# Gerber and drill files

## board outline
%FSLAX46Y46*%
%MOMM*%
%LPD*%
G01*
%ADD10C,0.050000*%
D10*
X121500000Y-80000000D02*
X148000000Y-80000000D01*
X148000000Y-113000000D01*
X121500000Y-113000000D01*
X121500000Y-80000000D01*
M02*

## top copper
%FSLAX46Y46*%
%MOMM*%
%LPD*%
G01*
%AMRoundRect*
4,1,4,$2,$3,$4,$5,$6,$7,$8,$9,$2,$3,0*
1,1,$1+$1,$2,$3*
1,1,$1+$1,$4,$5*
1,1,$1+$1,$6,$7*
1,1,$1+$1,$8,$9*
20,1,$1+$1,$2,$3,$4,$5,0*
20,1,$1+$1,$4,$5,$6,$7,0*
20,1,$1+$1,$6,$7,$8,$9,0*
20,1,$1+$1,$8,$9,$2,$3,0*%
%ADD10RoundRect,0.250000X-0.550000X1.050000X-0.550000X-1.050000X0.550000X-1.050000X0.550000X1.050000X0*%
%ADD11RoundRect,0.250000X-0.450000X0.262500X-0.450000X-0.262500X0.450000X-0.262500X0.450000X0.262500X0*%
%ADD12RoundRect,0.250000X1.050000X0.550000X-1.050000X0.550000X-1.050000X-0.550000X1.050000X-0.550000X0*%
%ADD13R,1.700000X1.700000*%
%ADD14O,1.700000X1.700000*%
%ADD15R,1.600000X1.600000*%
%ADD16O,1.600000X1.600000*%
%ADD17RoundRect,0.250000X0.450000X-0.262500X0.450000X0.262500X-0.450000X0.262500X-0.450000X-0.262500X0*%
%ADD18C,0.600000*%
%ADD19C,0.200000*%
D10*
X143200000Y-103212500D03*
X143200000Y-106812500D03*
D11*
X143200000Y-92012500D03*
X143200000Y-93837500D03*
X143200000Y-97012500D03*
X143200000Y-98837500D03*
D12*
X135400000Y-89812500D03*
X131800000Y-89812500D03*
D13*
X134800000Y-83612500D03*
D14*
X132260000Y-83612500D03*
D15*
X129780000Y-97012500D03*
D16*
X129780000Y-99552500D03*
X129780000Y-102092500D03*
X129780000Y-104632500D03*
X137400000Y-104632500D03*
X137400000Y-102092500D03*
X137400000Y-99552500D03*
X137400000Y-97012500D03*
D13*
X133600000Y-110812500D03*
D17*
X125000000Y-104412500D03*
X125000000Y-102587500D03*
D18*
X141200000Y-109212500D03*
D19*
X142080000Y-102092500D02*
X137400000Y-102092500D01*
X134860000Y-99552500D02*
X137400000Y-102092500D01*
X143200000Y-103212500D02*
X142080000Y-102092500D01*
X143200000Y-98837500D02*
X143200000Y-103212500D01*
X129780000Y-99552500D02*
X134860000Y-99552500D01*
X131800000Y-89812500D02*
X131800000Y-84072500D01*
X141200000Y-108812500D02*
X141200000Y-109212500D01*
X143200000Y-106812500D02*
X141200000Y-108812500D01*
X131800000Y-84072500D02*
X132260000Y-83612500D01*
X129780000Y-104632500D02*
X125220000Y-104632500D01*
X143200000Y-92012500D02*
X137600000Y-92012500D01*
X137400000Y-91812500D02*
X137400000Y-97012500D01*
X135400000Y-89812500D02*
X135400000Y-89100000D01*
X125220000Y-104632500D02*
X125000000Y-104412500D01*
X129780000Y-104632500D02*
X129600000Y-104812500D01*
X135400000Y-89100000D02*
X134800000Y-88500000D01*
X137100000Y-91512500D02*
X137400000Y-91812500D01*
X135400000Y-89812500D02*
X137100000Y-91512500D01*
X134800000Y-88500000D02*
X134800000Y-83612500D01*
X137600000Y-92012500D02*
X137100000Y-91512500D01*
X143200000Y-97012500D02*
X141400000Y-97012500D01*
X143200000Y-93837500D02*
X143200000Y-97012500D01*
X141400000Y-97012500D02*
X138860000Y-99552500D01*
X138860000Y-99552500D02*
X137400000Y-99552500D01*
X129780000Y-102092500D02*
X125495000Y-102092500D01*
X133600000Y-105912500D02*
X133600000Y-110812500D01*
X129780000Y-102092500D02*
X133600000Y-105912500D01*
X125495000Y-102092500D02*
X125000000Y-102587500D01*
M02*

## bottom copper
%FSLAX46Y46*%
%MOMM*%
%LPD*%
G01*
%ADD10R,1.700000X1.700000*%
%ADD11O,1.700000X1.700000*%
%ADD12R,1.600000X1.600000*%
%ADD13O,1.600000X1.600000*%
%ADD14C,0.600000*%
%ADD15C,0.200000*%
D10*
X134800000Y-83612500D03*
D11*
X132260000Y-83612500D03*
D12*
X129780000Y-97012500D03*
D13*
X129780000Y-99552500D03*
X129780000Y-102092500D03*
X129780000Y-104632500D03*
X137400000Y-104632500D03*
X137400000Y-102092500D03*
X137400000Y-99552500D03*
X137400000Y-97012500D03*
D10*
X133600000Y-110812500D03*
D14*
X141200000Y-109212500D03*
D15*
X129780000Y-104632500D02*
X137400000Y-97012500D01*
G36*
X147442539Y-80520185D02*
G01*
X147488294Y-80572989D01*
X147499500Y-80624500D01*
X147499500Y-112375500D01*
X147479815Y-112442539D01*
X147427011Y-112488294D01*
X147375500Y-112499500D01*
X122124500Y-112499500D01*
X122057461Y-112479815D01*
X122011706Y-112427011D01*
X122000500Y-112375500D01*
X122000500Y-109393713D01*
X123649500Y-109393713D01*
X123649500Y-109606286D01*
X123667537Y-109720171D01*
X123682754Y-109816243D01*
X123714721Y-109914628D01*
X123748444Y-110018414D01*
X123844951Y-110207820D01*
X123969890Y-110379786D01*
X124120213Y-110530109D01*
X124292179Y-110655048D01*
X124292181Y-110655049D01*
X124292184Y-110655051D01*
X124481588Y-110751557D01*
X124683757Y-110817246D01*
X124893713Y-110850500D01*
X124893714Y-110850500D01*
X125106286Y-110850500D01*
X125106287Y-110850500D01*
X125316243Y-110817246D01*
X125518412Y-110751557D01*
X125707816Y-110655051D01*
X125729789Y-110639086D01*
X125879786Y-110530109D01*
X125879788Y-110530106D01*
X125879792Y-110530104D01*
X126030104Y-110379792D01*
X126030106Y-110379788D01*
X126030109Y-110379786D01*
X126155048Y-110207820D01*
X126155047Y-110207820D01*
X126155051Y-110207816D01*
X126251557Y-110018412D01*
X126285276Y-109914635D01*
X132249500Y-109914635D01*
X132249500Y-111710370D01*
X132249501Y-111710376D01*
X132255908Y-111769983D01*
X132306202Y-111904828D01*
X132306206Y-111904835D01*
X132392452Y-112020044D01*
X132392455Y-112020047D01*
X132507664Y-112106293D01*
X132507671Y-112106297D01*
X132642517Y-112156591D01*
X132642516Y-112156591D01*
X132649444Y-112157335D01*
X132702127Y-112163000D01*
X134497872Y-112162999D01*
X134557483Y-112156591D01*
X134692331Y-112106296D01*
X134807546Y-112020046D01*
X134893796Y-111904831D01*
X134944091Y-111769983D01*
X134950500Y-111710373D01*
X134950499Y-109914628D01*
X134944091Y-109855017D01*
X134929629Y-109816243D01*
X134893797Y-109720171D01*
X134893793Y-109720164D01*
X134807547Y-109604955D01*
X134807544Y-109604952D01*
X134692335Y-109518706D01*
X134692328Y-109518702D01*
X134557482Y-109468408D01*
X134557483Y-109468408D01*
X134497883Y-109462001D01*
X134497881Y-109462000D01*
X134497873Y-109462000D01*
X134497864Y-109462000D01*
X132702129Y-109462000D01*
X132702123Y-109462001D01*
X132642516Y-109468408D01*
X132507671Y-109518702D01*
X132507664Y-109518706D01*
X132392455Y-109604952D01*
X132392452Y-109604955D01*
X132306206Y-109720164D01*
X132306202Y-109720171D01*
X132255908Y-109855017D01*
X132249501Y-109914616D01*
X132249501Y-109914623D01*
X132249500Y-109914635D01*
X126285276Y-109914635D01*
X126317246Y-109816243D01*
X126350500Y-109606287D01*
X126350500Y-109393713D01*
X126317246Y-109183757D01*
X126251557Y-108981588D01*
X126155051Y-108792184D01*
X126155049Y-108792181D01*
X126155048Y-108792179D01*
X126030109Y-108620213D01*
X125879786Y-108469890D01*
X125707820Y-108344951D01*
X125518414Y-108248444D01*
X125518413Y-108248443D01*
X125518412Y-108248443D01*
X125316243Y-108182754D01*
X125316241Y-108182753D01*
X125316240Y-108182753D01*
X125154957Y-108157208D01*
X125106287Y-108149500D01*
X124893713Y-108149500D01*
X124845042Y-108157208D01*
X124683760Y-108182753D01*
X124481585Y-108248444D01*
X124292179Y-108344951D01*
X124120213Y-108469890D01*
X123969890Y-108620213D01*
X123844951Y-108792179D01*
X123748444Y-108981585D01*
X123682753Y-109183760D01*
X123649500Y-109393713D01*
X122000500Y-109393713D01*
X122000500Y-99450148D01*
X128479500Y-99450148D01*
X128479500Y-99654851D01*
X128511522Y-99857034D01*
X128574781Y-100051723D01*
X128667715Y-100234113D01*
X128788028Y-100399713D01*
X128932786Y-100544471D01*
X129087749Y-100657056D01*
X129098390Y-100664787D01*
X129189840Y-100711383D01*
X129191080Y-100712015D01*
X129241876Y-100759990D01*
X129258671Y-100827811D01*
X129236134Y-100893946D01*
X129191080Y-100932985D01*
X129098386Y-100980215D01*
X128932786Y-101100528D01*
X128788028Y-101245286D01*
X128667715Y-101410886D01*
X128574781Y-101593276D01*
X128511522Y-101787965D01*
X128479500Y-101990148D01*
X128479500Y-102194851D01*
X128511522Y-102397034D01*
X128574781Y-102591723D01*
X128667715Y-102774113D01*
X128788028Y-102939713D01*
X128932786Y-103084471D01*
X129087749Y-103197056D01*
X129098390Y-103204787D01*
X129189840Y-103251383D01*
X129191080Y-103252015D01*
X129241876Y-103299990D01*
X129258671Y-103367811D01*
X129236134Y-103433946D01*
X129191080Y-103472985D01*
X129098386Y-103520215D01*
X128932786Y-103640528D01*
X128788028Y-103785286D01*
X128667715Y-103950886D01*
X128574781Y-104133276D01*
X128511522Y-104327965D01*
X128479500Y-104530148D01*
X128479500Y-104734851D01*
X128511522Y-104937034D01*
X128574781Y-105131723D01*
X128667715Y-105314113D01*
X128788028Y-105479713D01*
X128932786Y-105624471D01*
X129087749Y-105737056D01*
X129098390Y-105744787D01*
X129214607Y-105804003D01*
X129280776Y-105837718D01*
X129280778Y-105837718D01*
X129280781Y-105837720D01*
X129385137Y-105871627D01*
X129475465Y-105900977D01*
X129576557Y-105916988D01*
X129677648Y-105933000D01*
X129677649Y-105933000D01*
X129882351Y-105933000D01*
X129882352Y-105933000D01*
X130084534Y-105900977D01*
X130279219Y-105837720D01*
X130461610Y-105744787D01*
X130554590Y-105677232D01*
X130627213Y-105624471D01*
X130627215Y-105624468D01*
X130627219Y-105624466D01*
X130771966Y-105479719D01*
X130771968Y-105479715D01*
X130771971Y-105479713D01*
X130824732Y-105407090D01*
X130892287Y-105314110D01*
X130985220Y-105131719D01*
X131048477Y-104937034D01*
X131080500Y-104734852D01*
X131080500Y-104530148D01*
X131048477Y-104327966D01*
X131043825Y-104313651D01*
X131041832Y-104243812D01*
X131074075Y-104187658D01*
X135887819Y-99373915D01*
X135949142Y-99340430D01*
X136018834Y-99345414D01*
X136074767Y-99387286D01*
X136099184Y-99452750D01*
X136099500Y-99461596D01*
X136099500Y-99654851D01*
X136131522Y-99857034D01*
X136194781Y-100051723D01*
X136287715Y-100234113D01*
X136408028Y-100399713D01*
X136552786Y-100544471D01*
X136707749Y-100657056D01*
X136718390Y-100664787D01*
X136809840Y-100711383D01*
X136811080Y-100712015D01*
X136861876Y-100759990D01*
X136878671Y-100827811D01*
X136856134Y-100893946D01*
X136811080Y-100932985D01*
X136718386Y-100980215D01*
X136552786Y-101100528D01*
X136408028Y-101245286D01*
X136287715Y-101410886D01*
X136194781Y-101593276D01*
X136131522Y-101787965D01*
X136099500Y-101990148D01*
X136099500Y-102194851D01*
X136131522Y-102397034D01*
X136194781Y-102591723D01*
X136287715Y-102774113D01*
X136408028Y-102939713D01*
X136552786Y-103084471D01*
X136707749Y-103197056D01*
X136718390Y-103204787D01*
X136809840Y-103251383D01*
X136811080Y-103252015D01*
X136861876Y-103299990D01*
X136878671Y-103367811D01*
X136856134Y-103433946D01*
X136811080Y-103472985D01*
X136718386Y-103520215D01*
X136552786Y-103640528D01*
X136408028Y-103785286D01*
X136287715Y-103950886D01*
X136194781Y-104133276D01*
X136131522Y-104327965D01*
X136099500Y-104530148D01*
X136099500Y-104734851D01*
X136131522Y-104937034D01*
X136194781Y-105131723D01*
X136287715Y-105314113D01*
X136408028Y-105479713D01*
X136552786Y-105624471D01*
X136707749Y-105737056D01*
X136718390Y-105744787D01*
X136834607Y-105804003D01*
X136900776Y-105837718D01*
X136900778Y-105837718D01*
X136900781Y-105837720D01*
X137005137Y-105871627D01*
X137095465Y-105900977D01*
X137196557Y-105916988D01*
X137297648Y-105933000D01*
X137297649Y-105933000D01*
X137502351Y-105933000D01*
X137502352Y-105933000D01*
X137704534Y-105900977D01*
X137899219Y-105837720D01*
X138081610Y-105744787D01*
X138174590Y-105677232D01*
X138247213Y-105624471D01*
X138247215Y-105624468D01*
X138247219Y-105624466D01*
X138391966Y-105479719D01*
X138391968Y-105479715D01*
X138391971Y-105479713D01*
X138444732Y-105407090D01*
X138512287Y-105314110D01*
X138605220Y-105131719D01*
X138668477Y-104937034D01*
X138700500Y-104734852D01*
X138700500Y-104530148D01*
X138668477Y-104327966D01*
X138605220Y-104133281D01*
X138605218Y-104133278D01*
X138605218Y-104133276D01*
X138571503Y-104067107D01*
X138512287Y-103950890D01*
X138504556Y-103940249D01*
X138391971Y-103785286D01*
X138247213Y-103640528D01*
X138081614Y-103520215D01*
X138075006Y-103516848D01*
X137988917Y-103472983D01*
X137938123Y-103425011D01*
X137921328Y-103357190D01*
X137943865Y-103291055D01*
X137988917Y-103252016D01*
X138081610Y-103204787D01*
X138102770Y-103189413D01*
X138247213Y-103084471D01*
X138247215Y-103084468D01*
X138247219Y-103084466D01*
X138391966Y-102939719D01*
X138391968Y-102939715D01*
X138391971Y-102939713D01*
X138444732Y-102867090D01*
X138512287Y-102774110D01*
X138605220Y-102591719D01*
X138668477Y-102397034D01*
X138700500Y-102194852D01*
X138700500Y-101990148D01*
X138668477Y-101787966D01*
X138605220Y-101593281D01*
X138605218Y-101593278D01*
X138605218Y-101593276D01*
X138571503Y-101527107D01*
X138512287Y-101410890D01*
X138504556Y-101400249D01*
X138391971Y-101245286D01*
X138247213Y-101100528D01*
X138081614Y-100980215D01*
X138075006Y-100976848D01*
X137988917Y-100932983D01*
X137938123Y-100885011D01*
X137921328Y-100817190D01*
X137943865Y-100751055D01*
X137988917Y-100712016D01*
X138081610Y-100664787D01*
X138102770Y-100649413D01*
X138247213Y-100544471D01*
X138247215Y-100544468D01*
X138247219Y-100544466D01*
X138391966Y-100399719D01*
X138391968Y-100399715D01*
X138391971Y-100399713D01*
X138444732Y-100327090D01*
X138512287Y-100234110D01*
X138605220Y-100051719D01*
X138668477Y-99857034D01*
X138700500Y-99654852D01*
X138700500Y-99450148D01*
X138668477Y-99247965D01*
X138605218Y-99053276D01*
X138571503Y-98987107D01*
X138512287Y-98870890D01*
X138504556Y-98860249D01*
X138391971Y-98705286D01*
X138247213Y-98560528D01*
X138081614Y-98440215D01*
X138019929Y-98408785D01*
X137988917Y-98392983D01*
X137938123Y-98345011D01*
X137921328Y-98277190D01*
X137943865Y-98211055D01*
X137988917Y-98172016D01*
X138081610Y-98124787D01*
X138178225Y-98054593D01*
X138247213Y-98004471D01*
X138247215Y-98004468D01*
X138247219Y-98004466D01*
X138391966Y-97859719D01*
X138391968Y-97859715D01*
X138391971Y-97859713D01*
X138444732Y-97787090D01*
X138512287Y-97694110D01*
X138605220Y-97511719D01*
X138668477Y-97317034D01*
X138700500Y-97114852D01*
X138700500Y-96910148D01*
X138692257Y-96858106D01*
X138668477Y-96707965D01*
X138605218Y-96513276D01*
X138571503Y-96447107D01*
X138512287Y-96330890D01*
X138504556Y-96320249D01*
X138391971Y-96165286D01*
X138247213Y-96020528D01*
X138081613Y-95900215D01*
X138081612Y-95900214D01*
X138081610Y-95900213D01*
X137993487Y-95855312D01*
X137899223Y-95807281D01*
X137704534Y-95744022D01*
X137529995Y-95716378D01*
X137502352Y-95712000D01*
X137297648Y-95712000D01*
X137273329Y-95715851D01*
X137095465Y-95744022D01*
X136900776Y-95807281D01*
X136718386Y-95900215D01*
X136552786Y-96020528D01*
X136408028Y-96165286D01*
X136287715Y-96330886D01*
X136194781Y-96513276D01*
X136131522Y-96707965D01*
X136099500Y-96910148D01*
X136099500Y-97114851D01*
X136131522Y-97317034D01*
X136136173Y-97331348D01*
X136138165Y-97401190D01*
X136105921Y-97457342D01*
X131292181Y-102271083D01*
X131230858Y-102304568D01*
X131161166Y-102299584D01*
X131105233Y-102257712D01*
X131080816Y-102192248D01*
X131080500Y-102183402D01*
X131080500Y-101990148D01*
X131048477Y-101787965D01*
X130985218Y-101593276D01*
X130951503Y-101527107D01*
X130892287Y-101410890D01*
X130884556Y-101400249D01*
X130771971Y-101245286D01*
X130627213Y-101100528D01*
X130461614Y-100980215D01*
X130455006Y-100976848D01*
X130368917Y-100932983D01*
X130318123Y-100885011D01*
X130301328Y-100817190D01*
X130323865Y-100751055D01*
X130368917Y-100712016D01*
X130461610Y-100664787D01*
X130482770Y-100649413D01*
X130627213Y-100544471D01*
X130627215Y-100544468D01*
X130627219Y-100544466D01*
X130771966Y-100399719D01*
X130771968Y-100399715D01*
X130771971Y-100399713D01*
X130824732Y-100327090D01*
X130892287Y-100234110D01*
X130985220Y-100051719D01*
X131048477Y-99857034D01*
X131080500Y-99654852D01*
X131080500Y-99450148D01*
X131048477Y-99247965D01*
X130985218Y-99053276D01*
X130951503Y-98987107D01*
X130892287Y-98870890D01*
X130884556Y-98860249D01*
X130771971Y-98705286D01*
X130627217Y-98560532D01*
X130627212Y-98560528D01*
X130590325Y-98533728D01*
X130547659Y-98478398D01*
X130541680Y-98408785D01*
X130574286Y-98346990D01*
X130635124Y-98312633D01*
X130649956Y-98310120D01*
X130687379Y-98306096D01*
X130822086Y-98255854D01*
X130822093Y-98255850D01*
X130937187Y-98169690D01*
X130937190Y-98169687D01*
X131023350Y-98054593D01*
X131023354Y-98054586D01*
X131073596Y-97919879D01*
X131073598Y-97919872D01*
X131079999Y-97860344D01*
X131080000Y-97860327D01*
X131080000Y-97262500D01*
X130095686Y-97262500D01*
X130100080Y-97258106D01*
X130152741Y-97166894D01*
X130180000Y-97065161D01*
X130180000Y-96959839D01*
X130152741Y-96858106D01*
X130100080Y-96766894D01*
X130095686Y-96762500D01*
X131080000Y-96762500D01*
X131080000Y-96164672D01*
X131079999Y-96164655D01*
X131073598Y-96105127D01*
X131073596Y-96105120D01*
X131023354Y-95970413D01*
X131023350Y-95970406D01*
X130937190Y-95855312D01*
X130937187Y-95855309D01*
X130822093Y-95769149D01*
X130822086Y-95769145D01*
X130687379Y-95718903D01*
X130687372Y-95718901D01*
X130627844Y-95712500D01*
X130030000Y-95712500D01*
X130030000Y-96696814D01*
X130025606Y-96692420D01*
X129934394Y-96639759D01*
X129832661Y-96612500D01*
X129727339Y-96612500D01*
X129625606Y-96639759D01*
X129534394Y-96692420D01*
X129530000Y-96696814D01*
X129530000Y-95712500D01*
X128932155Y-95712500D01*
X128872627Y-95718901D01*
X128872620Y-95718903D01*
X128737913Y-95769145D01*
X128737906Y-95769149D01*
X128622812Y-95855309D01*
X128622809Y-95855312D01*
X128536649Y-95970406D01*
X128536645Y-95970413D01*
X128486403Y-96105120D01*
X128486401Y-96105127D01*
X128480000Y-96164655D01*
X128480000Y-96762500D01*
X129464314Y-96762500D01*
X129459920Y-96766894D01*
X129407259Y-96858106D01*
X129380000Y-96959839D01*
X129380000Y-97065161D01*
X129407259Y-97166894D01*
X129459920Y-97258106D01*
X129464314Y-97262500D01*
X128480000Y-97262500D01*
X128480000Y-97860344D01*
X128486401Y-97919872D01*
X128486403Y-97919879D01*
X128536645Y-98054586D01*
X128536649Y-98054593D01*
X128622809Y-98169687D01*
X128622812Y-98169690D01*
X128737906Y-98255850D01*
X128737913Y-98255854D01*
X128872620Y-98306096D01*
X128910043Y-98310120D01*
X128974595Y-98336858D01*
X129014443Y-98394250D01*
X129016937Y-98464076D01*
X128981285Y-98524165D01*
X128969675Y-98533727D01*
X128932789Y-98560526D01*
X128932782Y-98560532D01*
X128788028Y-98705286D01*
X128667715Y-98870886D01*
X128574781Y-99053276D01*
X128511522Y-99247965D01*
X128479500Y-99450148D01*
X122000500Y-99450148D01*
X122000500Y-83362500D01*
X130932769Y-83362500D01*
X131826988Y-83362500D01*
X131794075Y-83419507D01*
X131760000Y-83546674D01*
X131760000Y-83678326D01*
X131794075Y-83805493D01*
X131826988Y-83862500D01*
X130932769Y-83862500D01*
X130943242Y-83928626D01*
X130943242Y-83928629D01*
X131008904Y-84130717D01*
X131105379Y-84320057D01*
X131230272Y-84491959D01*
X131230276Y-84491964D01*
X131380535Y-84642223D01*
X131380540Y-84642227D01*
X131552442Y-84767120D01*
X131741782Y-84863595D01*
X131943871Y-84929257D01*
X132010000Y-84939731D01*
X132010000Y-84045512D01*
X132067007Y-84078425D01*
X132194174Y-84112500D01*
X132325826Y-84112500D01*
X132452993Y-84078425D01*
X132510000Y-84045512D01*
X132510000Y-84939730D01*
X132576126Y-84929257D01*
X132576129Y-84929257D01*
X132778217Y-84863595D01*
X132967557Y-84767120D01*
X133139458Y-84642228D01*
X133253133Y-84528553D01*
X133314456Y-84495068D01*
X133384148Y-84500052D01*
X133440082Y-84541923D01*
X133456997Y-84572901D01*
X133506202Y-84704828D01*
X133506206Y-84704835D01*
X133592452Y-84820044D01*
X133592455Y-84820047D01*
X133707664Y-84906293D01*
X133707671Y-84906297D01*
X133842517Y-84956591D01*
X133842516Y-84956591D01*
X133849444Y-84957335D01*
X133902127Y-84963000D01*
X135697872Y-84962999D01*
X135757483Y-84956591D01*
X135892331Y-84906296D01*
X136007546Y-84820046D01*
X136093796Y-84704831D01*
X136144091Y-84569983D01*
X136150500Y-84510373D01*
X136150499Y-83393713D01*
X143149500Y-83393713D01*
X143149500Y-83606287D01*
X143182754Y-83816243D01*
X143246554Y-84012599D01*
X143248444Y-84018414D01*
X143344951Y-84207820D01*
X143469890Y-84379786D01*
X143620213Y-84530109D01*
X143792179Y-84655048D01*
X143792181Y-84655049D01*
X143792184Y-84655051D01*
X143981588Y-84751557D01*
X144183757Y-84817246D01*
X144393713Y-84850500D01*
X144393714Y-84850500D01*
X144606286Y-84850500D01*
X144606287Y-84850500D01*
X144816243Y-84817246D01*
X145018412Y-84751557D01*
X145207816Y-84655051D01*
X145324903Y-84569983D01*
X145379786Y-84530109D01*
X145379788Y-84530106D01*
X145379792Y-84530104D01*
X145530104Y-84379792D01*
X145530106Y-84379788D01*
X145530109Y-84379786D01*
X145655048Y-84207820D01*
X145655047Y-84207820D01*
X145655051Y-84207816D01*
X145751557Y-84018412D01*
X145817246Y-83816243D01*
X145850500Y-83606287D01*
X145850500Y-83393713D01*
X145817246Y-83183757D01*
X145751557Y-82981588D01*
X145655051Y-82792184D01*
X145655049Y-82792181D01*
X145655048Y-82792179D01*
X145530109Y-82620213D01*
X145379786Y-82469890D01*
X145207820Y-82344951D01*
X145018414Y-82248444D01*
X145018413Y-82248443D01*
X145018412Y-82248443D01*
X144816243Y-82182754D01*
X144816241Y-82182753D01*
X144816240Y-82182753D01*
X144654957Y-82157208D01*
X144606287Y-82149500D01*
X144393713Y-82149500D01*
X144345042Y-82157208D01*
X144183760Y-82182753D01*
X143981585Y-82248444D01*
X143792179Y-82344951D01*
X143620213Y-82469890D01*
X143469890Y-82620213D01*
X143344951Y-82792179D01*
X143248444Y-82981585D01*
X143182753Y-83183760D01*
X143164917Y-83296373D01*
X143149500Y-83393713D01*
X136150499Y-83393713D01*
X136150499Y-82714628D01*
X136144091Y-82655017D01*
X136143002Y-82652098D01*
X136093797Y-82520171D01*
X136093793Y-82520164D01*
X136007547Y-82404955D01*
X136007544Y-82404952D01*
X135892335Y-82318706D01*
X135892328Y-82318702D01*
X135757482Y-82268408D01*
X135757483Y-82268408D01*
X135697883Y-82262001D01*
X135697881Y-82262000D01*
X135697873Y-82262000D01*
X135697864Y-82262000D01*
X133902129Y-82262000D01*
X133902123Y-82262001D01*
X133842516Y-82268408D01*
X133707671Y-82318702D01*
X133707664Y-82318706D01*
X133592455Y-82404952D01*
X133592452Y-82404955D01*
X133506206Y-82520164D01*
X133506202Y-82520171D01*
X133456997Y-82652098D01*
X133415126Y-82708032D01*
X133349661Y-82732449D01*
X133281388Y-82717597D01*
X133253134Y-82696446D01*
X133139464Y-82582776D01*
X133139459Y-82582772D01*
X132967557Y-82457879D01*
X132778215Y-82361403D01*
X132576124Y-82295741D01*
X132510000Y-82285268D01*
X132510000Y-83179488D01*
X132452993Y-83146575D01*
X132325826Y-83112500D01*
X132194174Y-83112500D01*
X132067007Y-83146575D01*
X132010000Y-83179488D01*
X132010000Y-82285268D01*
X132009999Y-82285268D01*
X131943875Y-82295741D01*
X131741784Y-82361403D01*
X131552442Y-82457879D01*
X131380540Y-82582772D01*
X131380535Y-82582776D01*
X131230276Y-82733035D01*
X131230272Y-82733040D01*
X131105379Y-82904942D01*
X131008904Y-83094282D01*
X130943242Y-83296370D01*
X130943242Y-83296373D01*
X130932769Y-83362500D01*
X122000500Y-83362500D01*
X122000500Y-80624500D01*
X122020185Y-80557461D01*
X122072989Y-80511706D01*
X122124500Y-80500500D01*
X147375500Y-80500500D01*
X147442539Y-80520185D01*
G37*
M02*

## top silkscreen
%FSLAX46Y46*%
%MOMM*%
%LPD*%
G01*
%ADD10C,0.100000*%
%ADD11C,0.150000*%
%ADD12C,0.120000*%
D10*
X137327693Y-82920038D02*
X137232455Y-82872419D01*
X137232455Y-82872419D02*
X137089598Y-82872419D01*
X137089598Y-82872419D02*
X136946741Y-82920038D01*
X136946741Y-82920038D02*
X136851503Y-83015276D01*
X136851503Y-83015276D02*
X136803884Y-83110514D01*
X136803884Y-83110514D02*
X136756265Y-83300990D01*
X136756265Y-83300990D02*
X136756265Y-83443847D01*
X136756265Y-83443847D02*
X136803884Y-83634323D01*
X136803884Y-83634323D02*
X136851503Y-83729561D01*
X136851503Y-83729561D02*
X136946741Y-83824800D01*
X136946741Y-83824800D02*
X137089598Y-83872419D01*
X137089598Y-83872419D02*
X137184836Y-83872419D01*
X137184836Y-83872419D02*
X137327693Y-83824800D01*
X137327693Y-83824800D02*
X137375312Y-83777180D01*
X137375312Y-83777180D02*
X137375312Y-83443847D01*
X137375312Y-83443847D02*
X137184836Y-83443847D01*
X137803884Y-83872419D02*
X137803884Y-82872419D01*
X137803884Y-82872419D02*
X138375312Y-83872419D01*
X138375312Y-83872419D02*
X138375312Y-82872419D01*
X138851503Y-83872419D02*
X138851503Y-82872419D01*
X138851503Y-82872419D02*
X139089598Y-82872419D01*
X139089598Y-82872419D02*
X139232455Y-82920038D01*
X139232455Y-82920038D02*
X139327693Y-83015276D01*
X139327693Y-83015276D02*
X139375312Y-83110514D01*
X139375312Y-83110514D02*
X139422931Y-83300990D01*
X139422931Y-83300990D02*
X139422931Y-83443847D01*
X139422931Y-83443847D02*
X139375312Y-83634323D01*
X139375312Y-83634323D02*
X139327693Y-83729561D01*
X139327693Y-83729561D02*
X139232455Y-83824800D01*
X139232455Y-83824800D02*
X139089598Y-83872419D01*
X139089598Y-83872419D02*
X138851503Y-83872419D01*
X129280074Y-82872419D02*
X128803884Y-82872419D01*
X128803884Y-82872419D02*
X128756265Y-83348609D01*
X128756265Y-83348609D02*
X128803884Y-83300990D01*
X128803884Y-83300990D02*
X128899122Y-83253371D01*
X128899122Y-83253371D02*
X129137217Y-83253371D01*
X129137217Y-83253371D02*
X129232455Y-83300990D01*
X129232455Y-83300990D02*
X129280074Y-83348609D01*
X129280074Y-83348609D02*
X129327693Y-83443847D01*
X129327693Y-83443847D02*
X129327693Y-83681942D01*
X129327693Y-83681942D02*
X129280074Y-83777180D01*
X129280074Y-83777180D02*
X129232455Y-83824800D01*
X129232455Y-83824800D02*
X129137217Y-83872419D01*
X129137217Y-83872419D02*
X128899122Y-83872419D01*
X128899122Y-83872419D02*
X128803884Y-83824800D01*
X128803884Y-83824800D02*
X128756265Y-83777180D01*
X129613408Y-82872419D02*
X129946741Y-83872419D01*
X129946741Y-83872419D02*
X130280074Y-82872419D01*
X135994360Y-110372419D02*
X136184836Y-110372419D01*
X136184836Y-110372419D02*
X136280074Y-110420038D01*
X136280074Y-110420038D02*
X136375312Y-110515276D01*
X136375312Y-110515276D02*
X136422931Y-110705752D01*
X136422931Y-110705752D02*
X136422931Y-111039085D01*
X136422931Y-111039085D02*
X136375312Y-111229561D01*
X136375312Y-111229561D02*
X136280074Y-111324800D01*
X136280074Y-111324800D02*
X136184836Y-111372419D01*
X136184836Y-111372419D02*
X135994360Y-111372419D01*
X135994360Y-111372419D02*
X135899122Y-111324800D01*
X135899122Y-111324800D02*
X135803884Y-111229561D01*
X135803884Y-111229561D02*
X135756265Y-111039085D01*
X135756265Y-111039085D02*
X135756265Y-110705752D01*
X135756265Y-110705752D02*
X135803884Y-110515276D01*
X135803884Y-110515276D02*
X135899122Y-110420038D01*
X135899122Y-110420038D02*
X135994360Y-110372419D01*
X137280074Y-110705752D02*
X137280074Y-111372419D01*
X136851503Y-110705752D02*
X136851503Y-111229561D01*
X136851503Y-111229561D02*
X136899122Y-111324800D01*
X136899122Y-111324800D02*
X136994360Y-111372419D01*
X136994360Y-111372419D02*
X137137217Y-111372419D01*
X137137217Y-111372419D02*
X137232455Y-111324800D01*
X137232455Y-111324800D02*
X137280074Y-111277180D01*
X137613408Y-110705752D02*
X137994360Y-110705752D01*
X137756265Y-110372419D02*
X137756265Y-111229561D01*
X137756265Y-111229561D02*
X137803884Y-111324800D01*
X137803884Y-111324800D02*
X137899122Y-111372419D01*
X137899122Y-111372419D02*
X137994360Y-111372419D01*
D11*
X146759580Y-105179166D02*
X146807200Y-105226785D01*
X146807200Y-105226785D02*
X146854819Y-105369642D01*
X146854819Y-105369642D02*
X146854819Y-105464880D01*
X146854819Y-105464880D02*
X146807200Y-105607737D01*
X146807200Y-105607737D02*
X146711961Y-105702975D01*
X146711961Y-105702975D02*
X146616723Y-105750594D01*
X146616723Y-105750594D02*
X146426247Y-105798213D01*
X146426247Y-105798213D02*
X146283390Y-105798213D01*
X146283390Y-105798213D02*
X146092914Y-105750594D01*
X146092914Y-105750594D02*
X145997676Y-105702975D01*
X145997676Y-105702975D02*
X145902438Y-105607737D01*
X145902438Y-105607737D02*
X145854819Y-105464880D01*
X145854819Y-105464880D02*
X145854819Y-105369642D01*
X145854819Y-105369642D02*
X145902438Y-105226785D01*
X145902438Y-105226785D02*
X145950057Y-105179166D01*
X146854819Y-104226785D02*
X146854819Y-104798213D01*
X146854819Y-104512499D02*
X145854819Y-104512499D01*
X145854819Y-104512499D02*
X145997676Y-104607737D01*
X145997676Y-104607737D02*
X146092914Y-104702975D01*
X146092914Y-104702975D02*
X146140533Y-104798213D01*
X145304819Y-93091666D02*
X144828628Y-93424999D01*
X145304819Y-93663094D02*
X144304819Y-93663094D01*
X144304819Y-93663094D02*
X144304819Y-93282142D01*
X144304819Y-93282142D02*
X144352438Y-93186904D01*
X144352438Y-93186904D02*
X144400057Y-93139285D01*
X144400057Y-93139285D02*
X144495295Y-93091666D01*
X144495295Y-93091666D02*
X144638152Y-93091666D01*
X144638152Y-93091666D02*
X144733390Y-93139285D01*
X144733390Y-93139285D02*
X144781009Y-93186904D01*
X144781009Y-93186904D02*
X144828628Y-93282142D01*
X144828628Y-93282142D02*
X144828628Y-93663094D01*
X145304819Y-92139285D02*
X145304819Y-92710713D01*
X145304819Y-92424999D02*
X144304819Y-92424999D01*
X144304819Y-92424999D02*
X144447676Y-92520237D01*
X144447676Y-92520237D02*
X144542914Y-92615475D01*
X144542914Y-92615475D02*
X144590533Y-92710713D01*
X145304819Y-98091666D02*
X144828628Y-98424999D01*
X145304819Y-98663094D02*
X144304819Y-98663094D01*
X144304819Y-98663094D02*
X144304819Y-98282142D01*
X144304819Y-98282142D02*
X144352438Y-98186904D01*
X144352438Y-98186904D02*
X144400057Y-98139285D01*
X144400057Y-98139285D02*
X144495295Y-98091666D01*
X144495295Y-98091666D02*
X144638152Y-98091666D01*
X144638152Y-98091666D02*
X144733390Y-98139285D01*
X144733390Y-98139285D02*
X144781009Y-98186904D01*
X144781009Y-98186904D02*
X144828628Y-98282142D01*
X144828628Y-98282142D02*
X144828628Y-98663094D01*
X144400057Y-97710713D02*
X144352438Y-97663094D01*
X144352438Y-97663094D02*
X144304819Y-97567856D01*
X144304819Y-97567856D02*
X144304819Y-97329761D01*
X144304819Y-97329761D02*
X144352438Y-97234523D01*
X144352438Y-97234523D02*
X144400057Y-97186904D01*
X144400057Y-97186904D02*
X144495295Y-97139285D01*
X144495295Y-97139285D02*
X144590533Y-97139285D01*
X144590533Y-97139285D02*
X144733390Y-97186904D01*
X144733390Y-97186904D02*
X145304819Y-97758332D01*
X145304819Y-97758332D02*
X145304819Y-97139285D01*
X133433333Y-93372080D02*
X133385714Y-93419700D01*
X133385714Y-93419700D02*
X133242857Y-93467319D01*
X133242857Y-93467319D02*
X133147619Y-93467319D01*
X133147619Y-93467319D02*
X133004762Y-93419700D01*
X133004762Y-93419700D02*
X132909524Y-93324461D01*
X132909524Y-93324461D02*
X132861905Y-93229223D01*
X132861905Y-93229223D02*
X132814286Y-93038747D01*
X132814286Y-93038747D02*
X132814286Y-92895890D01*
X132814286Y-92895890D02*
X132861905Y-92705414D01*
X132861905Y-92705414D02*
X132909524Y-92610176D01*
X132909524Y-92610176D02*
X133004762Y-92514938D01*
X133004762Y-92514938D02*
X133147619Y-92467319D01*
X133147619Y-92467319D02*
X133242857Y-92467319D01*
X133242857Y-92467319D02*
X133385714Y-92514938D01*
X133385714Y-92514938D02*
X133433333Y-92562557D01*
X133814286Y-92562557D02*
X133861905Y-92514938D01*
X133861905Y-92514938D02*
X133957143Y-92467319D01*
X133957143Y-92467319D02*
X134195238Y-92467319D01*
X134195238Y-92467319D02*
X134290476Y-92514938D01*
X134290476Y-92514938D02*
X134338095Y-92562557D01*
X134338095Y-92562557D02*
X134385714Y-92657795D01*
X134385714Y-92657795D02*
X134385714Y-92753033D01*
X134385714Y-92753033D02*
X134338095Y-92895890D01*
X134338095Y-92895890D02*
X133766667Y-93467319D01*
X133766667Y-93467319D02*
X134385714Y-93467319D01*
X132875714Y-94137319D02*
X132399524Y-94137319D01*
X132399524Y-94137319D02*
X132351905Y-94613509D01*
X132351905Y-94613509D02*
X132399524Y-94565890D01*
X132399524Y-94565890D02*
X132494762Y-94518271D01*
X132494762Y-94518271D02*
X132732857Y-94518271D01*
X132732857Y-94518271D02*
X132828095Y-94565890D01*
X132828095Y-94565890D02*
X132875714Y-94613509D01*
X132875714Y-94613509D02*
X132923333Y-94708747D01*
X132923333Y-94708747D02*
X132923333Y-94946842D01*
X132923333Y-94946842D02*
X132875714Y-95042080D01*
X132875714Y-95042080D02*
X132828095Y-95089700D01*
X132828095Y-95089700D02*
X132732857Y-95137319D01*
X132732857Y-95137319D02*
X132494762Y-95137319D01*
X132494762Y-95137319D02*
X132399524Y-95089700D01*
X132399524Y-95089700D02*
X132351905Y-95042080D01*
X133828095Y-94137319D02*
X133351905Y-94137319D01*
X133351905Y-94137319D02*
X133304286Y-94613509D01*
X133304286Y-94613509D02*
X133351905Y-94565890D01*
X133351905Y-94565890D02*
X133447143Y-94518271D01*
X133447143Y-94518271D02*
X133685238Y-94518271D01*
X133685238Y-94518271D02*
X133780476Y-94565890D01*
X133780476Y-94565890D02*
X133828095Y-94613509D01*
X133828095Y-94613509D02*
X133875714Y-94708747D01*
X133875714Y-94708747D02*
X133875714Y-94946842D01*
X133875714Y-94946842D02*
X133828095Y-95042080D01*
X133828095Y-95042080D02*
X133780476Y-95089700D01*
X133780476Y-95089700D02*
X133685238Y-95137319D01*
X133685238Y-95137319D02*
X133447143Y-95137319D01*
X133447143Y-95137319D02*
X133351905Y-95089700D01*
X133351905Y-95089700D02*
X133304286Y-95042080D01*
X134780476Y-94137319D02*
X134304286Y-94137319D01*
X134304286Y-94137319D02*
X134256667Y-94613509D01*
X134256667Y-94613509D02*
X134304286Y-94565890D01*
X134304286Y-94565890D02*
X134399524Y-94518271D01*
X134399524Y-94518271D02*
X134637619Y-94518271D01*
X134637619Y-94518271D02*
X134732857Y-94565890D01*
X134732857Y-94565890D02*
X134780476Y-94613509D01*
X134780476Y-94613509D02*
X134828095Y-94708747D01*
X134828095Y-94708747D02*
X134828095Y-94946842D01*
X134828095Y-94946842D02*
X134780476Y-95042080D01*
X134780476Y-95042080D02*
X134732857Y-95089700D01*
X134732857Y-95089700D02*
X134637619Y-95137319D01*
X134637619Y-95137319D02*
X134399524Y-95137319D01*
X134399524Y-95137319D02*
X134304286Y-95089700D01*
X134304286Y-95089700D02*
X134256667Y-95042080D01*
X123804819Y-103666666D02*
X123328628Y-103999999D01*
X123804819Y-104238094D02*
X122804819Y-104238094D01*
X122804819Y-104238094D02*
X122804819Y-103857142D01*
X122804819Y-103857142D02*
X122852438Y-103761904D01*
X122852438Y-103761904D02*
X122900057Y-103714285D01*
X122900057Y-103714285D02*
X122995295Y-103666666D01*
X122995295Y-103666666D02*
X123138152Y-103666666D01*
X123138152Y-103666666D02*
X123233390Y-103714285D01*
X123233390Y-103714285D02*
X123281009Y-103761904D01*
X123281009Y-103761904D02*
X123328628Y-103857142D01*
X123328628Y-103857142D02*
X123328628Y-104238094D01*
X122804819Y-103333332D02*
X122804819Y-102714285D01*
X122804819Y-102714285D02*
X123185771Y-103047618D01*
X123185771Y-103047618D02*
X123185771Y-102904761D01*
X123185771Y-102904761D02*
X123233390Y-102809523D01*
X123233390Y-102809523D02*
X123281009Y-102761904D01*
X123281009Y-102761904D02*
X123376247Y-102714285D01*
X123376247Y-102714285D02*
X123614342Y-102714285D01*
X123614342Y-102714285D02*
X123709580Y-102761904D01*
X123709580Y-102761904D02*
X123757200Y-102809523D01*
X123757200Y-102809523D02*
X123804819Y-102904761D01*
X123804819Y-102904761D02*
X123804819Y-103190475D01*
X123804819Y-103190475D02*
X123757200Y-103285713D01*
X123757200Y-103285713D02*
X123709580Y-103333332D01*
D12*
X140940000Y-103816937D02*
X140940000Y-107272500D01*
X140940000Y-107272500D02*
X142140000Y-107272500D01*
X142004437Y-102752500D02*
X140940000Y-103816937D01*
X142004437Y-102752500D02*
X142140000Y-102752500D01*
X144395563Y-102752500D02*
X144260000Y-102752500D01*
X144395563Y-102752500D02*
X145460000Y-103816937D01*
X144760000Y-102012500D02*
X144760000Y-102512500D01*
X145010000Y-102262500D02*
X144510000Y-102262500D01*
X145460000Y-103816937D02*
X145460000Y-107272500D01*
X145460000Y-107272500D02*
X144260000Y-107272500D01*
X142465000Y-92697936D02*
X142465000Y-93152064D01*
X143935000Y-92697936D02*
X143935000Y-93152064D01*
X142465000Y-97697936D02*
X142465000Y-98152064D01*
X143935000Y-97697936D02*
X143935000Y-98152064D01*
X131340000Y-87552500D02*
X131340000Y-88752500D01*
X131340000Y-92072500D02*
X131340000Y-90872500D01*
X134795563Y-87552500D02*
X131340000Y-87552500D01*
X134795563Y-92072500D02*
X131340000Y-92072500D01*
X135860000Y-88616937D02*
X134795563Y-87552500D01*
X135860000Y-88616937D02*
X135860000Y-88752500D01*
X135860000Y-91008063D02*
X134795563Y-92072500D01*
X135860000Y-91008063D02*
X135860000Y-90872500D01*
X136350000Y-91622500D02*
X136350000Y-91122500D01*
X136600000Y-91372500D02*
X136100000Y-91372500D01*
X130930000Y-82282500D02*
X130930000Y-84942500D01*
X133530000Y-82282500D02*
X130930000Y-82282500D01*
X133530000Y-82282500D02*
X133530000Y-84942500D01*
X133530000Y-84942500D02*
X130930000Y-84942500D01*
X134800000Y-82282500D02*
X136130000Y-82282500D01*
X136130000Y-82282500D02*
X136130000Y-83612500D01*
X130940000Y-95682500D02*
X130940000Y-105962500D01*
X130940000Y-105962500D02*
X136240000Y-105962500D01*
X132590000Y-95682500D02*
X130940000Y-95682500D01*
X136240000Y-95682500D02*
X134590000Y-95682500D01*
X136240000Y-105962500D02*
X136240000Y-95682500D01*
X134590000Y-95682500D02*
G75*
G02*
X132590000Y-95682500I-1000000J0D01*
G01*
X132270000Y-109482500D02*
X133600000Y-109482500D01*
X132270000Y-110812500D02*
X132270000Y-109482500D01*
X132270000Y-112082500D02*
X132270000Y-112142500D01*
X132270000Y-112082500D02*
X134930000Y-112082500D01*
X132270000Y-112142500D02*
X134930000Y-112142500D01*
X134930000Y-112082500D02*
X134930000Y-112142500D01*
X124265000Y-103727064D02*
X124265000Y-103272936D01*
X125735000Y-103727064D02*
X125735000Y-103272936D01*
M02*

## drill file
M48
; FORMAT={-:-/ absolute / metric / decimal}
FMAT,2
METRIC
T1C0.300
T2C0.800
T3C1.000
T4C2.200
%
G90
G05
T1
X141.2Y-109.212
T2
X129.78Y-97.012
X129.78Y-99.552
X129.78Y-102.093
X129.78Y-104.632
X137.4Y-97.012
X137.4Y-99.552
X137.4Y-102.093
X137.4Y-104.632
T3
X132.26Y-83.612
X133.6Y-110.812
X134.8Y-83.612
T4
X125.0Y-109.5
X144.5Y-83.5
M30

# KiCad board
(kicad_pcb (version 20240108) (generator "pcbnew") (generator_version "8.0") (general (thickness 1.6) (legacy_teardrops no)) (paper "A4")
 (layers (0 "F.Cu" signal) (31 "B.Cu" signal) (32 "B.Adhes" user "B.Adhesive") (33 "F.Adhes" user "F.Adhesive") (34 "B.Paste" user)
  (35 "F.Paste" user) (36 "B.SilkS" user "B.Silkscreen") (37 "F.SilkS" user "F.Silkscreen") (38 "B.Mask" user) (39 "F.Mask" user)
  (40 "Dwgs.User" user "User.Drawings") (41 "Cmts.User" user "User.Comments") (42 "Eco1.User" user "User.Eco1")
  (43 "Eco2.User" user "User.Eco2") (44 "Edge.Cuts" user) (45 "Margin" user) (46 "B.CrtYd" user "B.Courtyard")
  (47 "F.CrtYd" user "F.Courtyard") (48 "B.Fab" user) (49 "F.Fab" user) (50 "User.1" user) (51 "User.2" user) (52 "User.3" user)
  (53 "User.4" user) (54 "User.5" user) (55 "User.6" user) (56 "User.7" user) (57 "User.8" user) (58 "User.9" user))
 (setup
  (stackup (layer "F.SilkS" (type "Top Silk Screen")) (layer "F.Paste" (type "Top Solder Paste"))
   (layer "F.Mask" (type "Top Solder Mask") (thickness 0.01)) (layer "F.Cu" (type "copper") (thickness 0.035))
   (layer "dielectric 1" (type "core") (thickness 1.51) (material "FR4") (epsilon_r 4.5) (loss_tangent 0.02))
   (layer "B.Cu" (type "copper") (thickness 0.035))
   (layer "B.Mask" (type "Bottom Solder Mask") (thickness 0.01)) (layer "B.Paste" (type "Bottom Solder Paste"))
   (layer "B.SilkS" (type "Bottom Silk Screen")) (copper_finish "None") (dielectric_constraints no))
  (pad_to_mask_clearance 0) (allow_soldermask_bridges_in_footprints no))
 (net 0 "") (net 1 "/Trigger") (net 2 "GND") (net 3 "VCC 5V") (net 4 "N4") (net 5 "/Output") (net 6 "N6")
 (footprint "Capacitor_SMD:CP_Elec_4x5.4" (layer "F.Cu") (at 143.2 105.0125 -90)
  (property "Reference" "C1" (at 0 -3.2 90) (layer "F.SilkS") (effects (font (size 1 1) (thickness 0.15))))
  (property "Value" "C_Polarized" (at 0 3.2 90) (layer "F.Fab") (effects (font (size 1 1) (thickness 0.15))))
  (fp_line (start -1.195563 2.26) (end 2.26 2.26) (stroke (width 0.12) (type solid)) (layer "F.SilkS"))
  (fp_line (start 2.26 2.26) (end 2.26 1.06) (stroke (width 0.12) (type solid)) (layer "F.SilkS"))
  (fp_line (start -2.26 1.195563) (end -1.195563 2.26) (stroke (width 0.12) (type solid)) (layer "F.SilkS"))
  (fp_line (start -2.26 1.195563) (end -2.26 1.06) (stroke (width 0.12) (type solid)) (layer "F.SilkS"))
  (fp_line (start -2.26 -1.195563) (end -2.26 -1.06) (stroke (width 0.12) (type solid)) (layer "F.SilkS"))
  (fp_line (start -2.26 -1.195563) (end -1.195563 -2.26) (stroke (width 0.12) (type solid)) (layer "F.SilkS"))
  (fp_line (start -3 -1.56) (end -2.5 -1.56) (stroke (width 0.12) (type solid)) (layer "F.SilkS"))
  (fp_line (start -2.75 -1.81) (end -2.75 -1.31) (stroke (width 0.12) (type solid)) (layer "F.SilkS"))
  (fp_line (start -1.195563 -2.26) (end 2.26 -2.26) (stroke (width 0.12) (type solid)) (layer "F.SilkS"))
  (fp_line (start 2.26 -2.26) (end 2.26 -1.06) (stroke (width 0.12) (type solid)) (layer "F.SilkS"))
  (pad "1" smd roundrect (at -1.8 0 270) (size 2.6 1.6) (layers "F.Cu" "F.Paste" "F.Mask") (roundrect_rratio 0.15625) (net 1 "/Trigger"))
  (pad "2" smd roundrect (at 1.8 0 270) (size 2.6 1.6) (layers "F.Cu" "F.Paste" "F.Mask") (roundrect_rratio 0.15625) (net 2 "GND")))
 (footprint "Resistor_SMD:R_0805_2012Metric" (layer "F.Cu") (at 143.2 92.925 -90)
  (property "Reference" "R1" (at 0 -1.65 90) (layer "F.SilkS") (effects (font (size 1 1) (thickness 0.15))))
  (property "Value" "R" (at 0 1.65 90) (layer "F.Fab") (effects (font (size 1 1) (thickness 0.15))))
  (fp_line (start -0.227064 0.735) (end 0.227064 0.735) (stroke (width 0.12) (type solid)) (layer "F.SilkS"))
  (fp_line (start -0.227064 -0.735) (end 0.227064 -0.735) (stroke (width 0.12) (type solid)) (layer "F.SilkS"))
  (pad "1" smd roundrect (at -0.9125 0 270) (size 1.025 1.4) (layers "F.Cu" "F.Paste" "F.Mask") (roundrect_rratio 0.243902) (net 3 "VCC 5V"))
  (pad "2" smd roundrect (at 0.9125 0 270) (size 1.025 1.4) (layers "F.Cu" "F.Paste" "F.Mask") (roundrect_rratio 0.243902) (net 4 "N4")))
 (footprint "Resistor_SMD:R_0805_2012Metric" (layer "F.Cu") (at 143.2 97.925 -90)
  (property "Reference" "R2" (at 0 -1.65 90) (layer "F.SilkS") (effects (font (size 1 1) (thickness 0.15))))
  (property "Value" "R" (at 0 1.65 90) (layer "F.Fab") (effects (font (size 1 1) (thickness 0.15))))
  (fp_line (start -0.227064 0.735) (end 0.227064 0.735) (stroke (width 0.12) (type solid)) (layer "F.SilkS"))
  (fp_line (start -0.227064 -0.735) (end 0.227064 -0.735) (stroke (width 0.12) (type solid)) (layer "F.SilkS"))
  (pad "1" smd roundrect (at -0.9125 0 270) (size 1.025 1.4) (layers "F.Cu" "F.Paste" "F.Mask") (roundrect_rratio 0.243902) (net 4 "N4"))
  (pad "2" smd roundrect (at 0.9125 0 270) (size 1.025 1.4) (layers "F.Cu" "F.Paste" "F.Mask") (roundrect_rratio 0.243902)
   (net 1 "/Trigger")))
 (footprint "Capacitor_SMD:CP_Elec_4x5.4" (layer "F.Cu") (at 133.6 89.8125 180)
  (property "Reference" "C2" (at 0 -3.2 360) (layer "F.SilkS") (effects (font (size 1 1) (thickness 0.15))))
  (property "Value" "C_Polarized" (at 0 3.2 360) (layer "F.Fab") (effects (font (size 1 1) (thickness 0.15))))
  (fp_line (start 2.26 2.26) (end 2.26 1.06) (stroke (width 0.12) (type solid)) (layer "F.SilkS"))
  (fp_line (start 2.26 -2.26) (end 2.26 -1.06) (stroke (width 0.12) (type solid)) (layer "F.SilkS"))
  (fp_line (start -1.195563 2.26) (end 2.26 2.26) (stroke (width 0.12) (type solid)) (layer "F.SilkS"))
  (fp_line (start -1.195563 -2.26) (end 2.26 -2.26) (stroke (width 0.12) (type solid)) (layer "F.SilkS"))
  (fp_line (start -2.26 1.195563) (end -1.195563 2.26) (stroke (width 0.12) (type solid)) (layer "F.SilkS"))
  (fp_line (start -2.26 1.195563) (end -2.26 1.06) (stroke (width 0.12) (type solid)) (layer "F.SilkS"))
  (fp_line (start -2.26 -1.195563) (end -1.195563 -2.26) (stroke (width 0.12) (type solid)) (layer "F.SilkS"))
  (fp_line (start -2.26 -1.195563) (end -2.26 -1.06) (stroke (width 0.12) (type solid)) (layer "F.SilkS"))
  (fp_line (start -2.75 -1.81) (end -2.75 -1.31) (stroke (width 0.12) (type solid)) (layer "F.SilkS"))
  (fp_line (start -3 -1.56) (end -2.5 -1.56) (stroke (width 0.12) (type solid)) (layer "F.SilkS"))
  (pad "1" smd roundrect (at -1.8 0 180) (size 2.6 1.6) (layers "F.Cu" "F.Paste" "F.Mask") (roundrect_rratio 0.15625) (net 3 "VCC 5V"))
  (pad "2" smd roundrect (at 1.8 0 180) (size 2.6 1.6) (layers "F.Cu" "F.Paste" "F.Mask") (roundrect_rratio 0.15625) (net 2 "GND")))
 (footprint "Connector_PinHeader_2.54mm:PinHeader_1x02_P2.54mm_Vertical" (layer "F.Cu") (at 134.8 83.6125 -90)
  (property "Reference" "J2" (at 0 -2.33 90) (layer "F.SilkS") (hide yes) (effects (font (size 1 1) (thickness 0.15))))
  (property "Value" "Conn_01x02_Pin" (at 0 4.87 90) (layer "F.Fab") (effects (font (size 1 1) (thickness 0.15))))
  (fp_line (start -1.33 3.87) (end 1.33 3.87) (stroke (width 0.12) (type solid)) (layer "F.SilkS"))
  (fp_line (start -1.33 1.27) (end -1.33 3.87) (stroke (width 0.12) (type solid)) (layer "F.SilkS"))
  (fp_line (start -1.33 1.27) (end 1.33 1.27) (stroke (width 0.12) (type solid)) (layer "F.SilkS"))
  (fp_line (start 1.33 1.27) (end 1.33 3.87) (stroke (width 0.12) (type solid)) (layer "F.SilkS"))
  (fp_line (start -1.33 0) (end -1.33 -1.33) (stroke (width 0.12) (type solid)) (layer "F.SilkS"))
  (fp_line (start -1.33 -1.33) (end 0 -1.33) (stroke (width 0.12) (type solid)) (layer "F.SilkS"))
  (pad "1" thru_hole rect (at 0 0 270) (size 1.7 1.7) (drill 1) (layers "*.Cu" "*.Mask") (remove_unused_layers no) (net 3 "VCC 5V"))
  (pad "2" thru_hole oval (at 0 2.54 270) (size 1.7 1.7) (drill 1) (layers "*.Cu" "*.Mask") (remove_unused_layers no) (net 2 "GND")))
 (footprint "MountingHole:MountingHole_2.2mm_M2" (layer "F.Cu") (at 125 109.5)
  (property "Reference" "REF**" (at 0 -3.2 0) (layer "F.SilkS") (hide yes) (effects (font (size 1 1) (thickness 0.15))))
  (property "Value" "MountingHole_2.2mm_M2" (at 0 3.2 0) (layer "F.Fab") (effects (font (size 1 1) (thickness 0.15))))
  (pad "" np_thru_hole circle (at 0 0) (size 2.2 2.2) (drill 2.2) (layers "F&B.Cu" "*.Mask")))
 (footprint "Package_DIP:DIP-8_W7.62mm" (layer "F.Cu") (at 129.78 97.0125)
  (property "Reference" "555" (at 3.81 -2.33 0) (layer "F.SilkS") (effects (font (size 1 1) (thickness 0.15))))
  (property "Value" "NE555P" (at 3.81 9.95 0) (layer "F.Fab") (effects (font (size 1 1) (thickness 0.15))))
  (fp_line (start 1.16 -1.33) (end 1.16 8.95) (stroke (width 0.12) (type solid)) (layer "F.SilkS"))
  (fp_line (start 1.16 8.95) (end 6.46 8.95) (stroke (width 0.12) (type solid)) (layer "F.SilkS"))
  (fp_line (start 2.81 -1.33) (end 1.16 -1.33) (stroke (width 0.12) (type solid)) (layer "F.SilkS"))
  (fp_line (start 6.46 -1.33) (end 4.81 -1.33) (stroke (width 0.12) (type solid)) (layer "F.SilkS"))
  (fp_line (start 6.46 8.95) (end 6.46 -1.33) (stroke (width 0.12) (type solid)) (layer "F.SilkS"))
  (fp_arc (start 4.81 -1.33) (mid 3.81 -0.33) (end 2.81 -1.33) (stroke (width 0.12) (type solid)) (layer "F.SilkS"))
  (pad "1" thru_hole rect (at 0 0) (size 1.6 1.6) (drill 0.8) (layers "*.Cu" "*.Mask") (remove_unused_layers no) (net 2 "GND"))
  (pad "2" thru_hole oval (at 0 2.54) (size 1.6 1.6) (drill 0.8) (layers "*.Cu" "*.Mask") (remove_unused_layers no) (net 1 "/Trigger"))
  (pad "3" thru_hole oval (at 0 5.08) (size 1.6 1.6) (drill 0.8) (layers "*.Cu" "*.Mask") (remove_unused_layers no) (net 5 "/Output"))
  (pad "4" thru_hole oval (at 0 7.62) (size 1.6 1.6) (drill 0.8) (layers "*.Cu" "*.Mask") (remove_unused_layers no) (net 3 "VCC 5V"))
  (pad "5" thru_hole oval (at 7.62 7.62) (size 1.6 1.6) (drill 0.8) (layers "*.Cu" "*.Mask") (remove_unused_layers no) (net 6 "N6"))
  (pad "6" thru_hole oval (at 7.62 5.08) (size 1.6 1.6) (drill 0.8) (layers "*.Cu" "*.Mask") (remove_unused_layers no) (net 1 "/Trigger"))
  (pad "7" thru_hole oval (at 7.62 2.54) (size 1.6 1.6) (drill 0.8) (layers "*.Cu" "*.Mask") (remove_unused_layers no) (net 4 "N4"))
  (pad "8" thru_hole oval (at 7.62 0) (size 1.6 1.6) (drill 0.8) (layers "*.Cu" "*.Mask") (remove_unused_layers no) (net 3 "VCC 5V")))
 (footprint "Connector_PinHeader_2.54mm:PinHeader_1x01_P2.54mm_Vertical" (layer "F.Cu") (at 133.6 110.8125)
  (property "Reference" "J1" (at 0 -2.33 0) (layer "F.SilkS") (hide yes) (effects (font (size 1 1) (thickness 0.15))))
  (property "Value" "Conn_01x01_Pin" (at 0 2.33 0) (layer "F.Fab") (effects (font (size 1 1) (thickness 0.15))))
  (fp_line (start -1.33 -1.33) (end 0 -1.33) (stroke (width 0.12) (type solid)) (layer "F.SilkS"))
  (fp_line (start -1.33 0) (end -1.33 -1.33) (stroke (width 0.12) (type solid)) (layer "F.SilkS"))
  (fp_line (start -1.33 1.27) (end -1.33 1.33) (stroke (width 0.12) (type solid)) (layer "F.SilkS"))
  (fp_line (start -1.33 1.27) (end 1.33 1.27) (stroke (width 0.12) (type solid)) (layer "F.SilkS"))
  (fp_line (start -1.33 1.33) (end 1.33 1.33) (stroke (width 0.12) (type solid)) (layer "F.SilkS"))
  (fp_line (start 1.33 1.27) (end 1.33 1.33) (stroke (width 0.12) (type solid)) (layer "F.SilkS"))
  (pad "1" thru_hole rect (at 0 0) (size 1.7 1.7) (drill 1) (layers "*.Cu" "*.Mask") (remove_unused_layers no) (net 5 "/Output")))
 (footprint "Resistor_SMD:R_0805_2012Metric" (layer "F.Cu") (at 125 103.5 90)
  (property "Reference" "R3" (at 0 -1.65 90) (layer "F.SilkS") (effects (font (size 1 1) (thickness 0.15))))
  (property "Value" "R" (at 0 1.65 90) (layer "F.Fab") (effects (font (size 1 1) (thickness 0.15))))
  (fp_line (start -0.227064 -0.735) (end 0.227064 -0.735) (stroke (width 0.12) (type solid)) (layer "F.SilkS"))
  (fp_line (start -0.227064 0.735) (end 0.227064 0.735) (stroke (width 0.12) (type solid)) (layer "F.SilkS"))
  (pad "1" smd roundrect (at -0.9125 0 90) (size 1.025 1.4) (layers "F.Cu" "F.Paste" "F.Mask") (roundrect_rratio 0.243902) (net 3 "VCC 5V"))
  (pad "2" smd roundrect (at 0.9125 0 90) (size 1.025 1.4) (layers "F.Cu" "F.Paste" "F.Mask") (roundrect_rratio 0.243902) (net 5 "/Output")))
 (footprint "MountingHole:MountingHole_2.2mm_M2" (layer "F.Cu") (at 144.5 83.5)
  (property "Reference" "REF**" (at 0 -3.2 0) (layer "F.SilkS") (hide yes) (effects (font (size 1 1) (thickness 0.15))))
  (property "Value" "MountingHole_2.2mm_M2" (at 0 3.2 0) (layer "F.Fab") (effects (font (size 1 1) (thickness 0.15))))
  (pad "" np_thru_hole circle (at 0 0) (size 2.2 2.2) (drill 2.2) (layers "*.Cu" "*.Mask")))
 (gr_rect (start 121.5 80) (end 148 113) (stroke (width 0.05) (type default)) (fill none) (layer "Edge.Cuts"))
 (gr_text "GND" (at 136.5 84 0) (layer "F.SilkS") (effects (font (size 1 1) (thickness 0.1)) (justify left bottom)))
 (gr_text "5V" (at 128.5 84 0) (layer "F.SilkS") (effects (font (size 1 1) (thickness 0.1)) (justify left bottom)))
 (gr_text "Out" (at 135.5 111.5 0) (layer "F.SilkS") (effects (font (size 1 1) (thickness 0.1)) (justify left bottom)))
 (segment (start 142.08 102.0925) (end 137.4 102.0925) (width 0.2) (layer "F.Cu") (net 1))
 (segment (start 134.86 99.5525) (end 137.4 102.0925) (width 0.2) (layer "F.Cu") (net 1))
 (segment (start 143.2 103.2125) (end 142.08 102.0925) (width 0.2) (layer "F.Cu") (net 1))
 (segment (start 143.2 98.8375) (end 143.2 103.2125) (width 0.2) (layer "F.Cu") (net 1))
 (segment (start 129.78 99.5525) (end 134.86 99.5525) (width 0.2) (layer "F.Cu") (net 1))
 (segment (start 131.8 89.8125) (end 131.8 84.0725) (width 0.2) (layer "F.Cu") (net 2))
 (segment (start 141.2 108.8125) (end 141.2 109.2125) (width 0.2) (layer "F.Cu") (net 2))
 (segment (start 143.2 106.8125) (end 141.2 108.8125) (width 0.2) (layer "F.Cu") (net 2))
 (segment (start 131.8 84.0725) (end 132.26 83.6125) (width 0.2) (layer "F.Cu") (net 2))
 (via (at 141.2 109.2125) (size 0.6) (drill 0.3) (layers "F.Cu" "B.Cu") (free yes) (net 2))
 (segment (start 129.78 104.6325) (end 125.22 104.6325) (width 0.2) (layer "F.Cu") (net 3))
 (segment (start 143.2 92.0125) (end 137.6 92.0125) (width 0.2) (layer "F.Cu") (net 3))
 (segment (start 137.4 91.8125) (end 137.4 97.0125) (width 0.2) (layer "F.Cu") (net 3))
 (segment (start 135.4 89.8125) (end 135.4 89.1) (width 0.2) (layer "F.Cu") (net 3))
 (segment (start 125.22 104.6325) (end 125 104.4125) (width 0.2) (layer "F.Cu") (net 3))
 (segment (start 129.78 104.6325) (end 129.6 104.8125) (width 0.2) (layer "F.Cu") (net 3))
 (segment (start 135.4 89.1) (end 134.8 88.5) (width 0.2) (layer "F.Cu") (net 3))
 (segment (start 137.1 91.5125) (end 137.4 91.8125) (width 0.2) (layer "F.Cu") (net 3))
 (segment (start 135.4 89.8125) (end 137.1 91.5125) (width 0.2) (layer "F.Cu") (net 3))
 (segment (start 134.8 88.5) (end 134.8 83.6125) (width 0.2) (layer "F.Cu") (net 3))
 (segment (start 137.6 92.0125) (end 137.1 91.5125) (width 0.2) (layer "F.Cu") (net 3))
 (segment (start 129.78 104.6325) (end 137.4 97.0125) (width 0.2) (layer "B.Cu") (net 3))
 (segment (start 143.2 97.0125) (end 141.4 97.0125) (width 0.2) (layer "F.Cu") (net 4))
 (segment (start 143.2 93.8375) (end 143.2 97.0125) (width 0.2) (layer "F.Cu") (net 4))
 (segment (start 141.4 97.0125) (end 138.86 99.5525) (width 0.2) (layer "F.Cu") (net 4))
 (segment (start 138.86 99.5525) (end 137.4 99.5525) (width 0.2) (layer "F.Cu") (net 4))
 (segment (start 129.78 102.0925) (end 125.495 102.0925) (width 0.2) (layer "F.Cu") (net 5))
 (segment (start 133.6 105.9125) (end 133.6 110.8125) (width 0.2) (layer "F.Cu") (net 5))
 (segment (start 129.78 102.0925) (end 133.6 105.9125) (width 0.2) (layer "F.Cu") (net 5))
 (segment (start 125.495 102.0925) (end 125 102.5875) (width 0.2) (layer "F.Cu") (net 5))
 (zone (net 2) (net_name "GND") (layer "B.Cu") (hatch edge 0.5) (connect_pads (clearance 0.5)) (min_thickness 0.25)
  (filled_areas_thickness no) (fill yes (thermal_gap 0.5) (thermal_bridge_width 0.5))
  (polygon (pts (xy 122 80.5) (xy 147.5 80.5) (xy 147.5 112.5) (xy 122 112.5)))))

